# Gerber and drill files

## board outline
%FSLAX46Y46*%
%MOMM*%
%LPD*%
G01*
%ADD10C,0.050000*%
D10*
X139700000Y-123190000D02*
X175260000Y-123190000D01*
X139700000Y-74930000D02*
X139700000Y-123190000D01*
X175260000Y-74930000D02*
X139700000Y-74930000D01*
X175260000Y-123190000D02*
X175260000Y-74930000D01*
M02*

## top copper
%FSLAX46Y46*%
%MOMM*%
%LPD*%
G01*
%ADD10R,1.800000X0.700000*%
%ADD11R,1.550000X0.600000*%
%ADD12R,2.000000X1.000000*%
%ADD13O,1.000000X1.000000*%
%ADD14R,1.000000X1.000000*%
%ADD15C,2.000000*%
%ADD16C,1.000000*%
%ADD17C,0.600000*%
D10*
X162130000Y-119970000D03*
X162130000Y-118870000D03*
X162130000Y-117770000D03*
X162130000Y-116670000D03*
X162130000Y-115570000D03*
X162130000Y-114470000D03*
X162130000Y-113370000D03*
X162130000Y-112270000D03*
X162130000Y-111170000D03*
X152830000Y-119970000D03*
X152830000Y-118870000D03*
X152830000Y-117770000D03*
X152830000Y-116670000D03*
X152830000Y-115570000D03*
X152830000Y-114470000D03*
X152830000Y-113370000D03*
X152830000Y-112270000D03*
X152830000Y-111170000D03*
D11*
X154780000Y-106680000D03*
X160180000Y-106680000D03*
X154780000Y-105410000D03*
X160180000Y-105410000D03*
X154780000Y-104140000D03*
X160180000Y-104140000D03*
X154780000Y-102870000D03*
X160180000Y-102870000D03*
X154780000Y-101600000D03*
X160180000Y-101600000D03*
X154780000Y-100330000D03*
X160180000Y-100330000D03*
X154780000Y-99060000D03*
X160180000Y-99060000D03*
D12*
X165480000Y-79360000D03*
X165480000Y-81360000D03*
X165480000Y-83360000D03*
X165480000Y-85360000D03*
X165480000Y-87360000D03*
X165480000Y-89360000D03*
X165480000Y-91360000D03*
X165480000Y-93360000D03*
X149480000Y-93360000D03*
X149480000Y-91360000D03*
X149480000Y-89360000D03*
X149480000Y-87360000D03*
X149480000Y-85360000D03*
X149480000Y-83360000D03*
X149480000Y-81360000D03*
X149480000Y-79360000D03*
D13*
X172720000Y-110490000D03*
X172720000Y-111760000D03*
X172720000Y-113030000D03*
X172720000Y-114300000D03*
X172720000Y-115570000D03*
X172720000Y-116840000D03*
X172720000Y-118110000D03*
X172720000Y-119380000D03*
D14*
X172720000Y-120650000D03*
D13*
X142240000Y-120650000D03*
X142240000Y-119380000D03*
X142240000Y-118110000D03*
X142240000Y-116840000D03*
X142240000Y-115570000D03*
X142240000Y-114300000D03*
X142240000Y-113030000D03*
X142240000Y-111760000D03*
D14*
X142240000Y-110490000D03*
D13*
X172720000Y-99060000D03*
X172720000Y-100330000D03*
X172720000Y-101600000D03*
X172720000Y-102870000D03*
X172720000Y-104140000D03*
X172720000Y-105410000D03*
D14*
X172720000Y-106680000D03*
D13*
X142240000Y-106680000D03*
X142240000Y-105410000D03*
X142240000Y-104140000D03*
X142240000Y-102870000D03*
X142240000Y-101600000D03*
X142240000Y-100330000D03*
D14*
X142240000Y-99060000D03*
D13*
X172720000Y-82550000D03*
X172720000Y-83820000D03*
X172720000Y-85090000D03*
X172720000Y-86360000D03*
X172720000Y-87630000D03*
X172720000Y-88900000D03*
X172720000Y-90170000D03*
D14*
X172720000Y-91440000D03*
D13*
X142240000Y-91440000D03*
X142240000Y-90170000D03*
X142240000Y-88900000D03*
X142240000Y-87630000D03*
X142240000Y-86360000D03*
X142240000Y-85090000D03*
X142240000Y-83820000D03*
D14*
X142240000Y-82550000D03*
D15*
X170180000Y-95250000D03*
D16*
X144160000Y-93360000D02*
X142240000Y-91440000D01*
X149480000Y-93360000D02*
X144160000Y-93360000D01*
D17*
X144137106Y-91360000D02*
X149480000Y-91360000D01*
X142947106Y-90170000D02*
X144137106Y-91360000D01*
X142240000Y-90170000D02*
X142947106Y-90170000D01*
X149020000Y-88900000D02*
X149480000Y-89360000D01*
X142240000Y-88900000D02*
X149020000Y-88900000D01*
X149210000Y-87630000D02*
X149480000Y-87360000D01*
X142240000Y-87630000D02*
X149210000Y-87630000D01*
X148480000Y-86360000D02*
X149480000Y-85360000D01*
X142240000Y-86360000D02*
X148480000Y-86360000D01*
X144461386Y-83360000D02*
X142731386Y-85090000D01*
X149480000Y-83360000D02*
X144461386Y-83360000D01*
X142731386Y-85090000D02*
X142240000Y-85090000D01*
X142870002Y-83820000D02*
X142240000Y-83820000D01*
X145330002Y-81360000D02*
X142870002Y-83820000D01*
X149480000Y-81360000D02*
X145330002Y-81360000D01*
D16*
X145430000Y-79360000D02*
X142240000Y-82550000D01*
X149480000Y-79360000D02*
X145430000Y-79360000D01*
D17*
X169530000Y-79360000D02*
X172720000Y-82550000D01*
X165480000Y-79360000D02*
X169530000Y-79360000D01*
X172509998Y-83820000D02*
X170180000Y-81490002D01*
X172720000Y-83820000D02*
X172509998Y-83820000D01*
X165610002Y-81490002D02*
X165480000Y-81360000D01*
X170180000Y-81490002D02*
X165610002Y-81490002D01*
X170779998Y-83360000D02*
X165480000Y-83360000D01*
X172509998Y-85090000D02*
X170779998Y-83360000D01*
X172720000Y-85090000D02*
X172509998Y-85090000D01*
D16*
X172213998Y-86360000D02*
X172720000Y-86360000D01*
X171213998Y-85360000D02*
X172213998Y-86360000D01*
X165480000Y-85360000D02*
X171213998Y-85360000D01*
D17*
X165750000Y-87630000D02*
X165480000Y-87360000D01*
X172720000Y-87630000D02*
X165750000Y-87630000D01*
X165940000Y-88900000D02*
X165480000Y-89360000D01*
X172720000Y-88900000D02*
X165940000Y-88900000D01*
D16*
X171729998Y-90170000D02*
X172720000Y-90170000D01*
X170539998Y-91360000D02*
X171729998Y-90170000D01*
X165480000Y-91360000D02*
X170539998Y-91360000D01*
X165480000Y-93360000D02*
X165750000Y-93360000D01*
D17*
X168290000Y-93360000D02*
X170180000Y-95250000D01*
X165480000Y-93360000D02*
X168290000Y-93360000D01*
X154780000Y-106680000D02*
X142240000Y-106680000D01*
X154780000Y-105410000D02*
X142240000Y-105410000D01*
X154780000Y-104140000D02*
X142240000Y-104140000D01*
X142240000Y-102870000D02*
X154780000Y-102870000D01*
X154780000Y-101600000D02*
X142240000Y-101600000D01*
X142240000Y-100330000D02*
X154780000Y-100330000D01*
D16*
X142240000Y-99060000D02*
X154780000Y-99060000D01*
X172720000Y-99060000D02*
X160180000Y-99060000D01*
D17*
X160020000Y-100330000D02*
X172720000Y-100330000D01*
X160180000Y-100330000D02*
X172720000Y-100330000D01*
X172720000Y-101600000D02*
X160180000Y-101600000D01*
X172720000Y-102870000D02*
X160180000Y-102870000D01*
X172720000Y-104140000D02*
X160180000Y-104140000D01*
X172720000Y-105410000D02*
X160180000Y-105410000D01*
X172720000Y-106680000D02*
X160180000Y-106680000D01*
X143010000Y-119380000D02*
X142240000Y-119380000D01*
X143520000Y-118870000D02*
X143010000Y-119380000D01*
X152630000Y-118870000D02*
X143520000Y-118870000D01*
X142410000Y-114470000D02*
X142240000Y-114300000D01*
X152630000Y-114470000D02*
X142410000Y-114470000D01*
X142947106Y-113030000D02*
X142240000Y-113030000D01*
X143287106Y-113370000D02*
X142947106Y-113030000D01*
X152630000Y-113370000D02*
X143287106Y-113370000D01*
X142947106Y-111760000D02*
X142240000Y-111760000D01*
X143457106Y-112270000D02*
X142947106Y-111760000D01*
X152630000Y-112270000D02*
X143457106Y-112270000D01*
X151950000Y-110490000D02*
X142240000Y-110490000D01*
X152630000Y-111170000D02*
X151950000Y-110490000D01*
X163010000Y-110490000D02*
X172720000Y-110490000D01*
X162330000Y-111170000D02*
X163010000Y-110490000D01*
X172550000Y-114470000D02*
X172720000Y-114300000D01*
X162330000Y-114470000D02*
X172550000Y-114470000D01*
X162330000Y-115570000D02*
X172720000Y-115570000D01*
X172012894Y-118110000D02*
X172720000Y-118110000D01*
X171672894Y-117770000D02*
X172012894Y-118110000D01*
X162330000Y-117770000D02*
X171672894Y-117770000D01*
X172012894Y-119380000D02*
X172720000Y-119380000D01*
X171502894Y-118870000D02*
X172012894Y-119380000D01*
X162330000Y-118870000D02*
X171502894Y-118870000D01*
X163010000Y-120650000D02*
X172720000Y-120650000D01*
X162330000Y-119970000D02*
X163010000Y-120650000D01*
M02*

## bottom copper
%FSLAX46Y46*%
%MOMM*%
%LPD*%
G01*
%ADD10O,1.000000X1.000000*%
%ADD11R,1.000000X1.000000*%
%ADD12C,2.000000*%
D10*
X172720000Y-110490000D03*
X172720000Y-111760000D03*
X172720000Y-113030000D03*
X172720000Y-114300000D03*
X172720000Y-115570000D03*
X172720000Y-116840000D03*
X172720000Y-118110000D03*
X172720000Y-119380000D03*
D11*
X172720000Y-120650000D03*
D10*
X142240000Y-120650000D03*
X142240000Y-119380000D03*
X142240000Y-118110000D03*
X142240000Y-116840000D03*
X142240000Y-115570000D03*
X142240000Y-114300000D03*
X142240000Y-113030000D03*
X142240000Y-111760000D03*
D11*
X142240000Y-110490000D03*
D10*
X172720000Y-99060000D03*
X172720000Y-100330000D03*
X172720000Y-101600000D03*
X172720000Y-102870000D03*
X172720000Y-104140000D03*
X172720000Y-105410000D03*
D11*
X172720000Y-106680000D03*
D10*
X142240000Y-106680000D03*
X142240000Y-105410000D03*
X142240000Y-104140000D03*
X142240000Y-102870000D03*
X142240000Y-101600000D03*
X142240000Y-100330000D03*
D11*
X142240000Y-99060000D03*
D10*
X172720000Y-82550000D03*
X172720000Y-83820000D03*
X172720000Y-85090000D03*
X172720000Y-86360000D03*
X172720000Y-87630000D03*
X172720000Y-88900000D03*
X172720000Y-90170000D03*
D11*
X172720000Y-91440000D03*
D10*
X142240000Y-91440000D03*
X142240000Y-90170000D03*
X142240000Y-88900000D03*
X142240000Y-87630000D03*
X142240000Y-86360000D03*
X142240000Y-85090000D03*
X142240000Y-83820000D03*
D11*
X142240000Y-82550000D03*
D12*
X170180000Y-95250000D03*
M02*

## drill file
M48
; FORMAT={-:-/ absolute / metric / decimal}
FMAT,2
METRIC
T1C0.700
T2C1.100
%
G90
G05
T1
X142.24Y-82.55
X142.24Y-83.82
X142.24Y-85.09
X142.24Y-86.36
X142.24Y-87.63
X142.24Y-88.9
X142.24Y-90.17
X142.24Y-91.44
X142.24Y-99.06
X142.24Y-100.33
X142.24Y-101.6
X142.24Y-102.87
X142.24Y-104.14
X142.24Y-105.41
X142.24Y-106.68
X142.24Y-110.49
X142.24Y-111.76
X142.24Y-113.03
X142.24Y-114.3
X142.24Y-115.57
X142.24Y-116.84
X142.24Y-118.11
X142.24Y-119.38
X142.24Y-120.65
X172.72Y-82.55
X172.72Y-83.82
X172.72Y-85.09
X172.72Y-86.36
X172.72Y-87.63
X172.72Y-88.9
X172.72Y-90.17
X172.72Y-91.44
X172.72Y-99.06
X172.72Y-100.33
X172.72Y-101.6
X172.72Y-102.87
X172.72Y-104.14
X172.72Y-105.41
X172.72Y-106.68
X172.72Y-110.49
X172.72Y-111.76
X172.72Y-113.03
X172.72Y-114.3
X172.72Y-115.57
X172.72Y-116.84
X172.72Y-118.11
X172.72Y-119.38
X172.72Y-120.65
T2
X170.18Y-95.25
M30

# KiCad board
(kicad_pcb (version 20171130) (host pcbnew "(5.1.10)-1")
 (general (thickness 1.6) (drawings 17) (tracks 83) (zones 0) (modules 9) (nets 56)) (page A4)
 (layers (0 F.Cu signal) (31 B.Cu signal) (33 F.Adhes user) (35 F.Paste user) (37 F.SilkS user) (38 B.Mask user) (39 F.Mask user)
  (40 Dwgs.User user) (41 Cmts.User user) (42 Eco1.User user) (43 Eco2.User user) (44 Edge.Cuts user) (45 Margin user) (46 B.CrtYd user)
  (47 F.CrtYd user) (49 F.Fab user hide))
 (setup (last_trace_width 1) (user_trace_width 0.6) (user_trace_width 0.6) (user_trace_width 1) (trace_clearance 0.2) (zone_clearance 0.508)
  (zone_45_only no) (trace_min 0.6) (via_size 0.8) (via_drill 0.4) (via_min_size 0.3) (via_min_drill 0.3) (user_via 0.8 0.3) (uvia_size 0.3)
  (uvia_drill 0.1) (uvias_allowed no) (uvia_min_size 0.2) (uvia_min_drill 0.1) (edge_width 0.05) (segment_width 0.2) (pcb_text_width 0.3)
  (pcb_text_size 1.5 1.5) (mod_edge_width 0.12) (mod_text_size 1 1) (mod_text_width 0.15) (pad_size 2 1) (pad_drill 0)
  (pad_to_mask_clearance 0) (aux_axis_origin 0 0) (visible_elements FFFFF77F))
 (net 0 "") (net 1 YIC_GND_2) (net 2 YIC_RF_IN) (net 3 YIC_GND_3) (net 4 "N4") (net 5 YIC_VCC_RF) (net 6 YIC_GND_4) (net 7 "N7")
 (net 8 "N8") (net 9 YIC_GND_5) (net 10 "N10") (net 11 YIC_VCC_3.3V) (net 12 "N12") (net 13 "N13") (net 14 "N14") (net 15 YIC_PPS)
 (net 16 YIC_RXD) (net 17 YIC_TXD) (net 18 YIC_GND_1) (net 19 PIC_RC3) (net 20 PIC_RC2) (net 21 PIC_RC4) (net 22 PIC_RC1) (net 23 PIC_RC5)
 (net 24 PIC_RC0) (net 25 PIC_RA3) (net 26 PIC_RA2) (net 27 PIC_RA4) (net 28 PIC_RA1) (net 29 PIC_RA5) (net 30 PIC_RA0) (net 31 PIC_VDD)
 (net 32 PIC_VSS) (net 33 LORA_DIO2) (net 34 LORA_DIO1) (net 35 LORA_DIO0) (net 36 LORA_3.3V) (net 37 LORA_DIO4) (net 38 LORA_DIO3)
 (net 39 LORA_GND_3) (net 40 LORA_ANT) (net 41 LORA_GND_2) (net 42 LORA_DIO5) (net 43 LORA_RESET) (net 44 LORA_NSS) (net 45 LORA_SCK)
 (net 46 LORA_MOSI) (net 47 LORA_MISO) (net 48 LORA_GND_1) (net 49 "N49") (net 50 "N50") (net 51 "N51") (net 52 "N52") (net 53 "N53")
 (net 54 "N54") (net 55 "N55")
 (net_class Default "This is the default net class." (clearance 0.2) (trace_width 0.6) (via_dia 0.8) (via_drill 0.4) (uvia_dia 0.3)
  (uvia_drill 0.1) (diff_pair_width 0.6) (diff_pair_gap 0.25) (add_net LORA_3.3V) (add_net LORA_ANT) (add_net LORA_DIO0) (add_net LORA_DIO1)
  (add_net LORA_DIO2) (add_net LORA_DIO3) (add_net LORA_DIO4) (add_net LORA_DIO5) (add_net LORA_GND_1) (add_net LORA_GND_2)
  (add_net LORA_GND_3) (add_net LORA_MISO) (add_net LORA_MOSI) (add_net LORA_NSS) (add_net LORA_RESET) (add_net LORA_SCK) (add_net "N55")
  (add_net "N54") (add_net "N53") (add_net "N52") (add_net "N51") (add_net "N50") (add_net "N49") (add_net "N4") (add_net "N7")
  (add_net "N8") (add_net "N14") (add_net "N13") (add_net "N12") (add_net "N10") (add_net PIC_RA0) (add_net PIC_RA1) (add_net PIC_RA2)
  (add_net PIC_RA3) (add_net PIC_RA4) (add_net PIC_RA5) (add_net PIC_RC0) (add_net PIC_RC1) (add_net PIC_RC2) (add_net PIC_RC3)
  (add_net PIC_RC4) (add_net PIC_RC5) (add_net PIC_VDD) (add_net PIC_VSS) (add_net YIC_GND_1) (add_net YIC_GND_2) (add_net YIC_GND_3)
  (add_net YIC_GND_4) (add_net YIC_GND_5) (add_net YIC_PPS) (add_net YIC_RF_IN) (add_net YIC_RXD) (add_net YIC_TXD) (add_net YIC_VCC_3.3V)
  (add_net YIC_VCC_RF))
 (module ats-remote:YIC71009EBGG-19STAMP (layer F.Cu) (at 157.48 115.57 270)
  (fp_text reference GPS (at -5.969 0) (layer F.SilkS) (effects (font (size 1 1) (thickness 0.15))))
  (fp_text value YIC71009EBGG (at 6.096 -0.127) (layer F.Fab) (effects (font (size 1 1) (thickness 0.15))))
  (pad 10 smd rect (at 4.4 -4.85 270) (size 0.7 1.8) (drill (offset 0 0.2)) (layers F.Cu F.Paste F.Mask) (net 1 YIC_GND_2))
  (pad 11 smd rect (at 3.3 -4.85 270) (size 0.7 1.8) (drill (offset 0 0.2)) (layers F.Cu F.Paste F.Mask) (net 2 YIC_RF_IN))
  (pad 12 smd rect (at 2.2 -4.85 270) (size 0.7 1.8) (drill (offset 0 0.2)) (layers F.Cu F.Paste F.Mask) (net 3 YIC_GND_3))
  (pad 13 smd rect (at 1.1 -4.85 270) (size 0.7 1.8) (drill (offset 0 0.2)) (layers F.Cu F.Paste F.Mask) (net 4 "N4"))
  (pad 14 smd rect (at 0 -4.85 270) (size 0.7 1.8) (drill (offset 0 0.2)) (layers F.Cu F.Paste F.Mask) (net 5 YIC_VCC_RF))
  (pad 15 smd rect (at -1.1 -4.85 270) (size 0.7 1.8) (drill (offset 0 0.2)) (layers F.Cu F.Paste F.Mask) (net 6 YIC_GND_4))
  (pad 16 smd rect (at -2.2 -4.85 270) (size 0.7 1.8) (drill (offset 0 0.2)) (layers F.Cu F.Paste F.Mask) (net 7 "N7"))
  (pad 17 smd rect (at -3.3 -4.85 270) (size 0.7 1.8) (drill (offset 0 0.2)) (layers F.Cu F.Paste F.Mask) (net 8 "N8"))
  (pad 18 smd rect (at -4.4 -4.85 270) (size 0.7 1.8) (drill (offset 0 0.2)) (layers F.Cu F.Paste F.Mask) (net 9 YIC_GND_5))
  (pad 9 smd rect (at 4.4 4.85 270) (size 0.7 1.8) (drill (offset 0 -0.2)) (layers F.Cu F.Paste F.Mask) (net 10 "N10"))
  (pad 8 smd rect (at 3.3 4.85 270) (size 0.7 1.8) (drill (offset 0 -0.2)) (layers F.Cu F.Paste F.Mask) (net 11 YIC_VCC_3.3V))
  (pad 7 smd rect (at 2.2 4.85 270) (size 0.7 1.8) (drill (offset 0 -0.2)) (layers F.Cu F.Paste F.Mask) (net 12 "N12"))
  (pad 6 smd rect (at 1.1 4.85 270) (size 0.7 1.8) (drill (offset 0 -0.2)) (layers F.Cu F.Paste F.Mask) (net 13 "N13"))
  (pad 5 smd rect (at 0 4.85 270) (size 0.7 1.8) (drill (offset 0 -0.2)) (layers F.Cu F.Paste F.Mask) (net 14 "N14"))
  (pad 4 smd rect (at -1.1 4.85 270) (size 0.7 1.8) (drill (offset 0 -0.2)) (layers F.Cu F.Paste F.Mask) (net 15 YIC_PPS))
  (pad 3 smd rect (at -2.2 4.85 270) (size 0.7 1.8) (drill (offset 0 -0.2)) (layers F.Cu F.Paste F.Mask) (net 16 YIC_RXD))
  (pad 2 smd rect (at -3.3 4.85 270) (size 0.7 1.8) (drill (offset 0 -0.2)) (layers F.Cu F.Paste F.Mask) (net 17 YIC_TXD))
  (pad 1 smd rect (at -4.4 4.85 270) (size 0.7 1.8) (drill (offset 0 -0.2)) (layers F.Cu F.Paste F.Mask) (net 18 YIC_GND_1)))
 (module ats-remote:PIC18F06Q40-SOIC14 (layer F.Cu) (at 157.48 102.87 270)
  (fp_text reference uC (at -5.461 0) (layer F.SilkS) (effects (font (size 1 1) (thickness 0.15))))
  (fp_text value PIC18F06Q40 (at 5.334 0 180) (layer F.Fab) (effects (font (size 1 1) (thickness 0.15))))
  (pad 7 smd rect (at 3.81 2.7 270) (size 0.6 1.55) (layers F.Cu F.Paste F.Mask) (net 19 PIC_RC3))
  (pad 8 smd rect (at 3.81 -2.7 270) (size 0.6 1.55) (layers F.Cu F.Paste F.Mask) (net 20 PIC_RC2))
  (pad 6 smd rect (at 2.54 2.7 270) (size 0.6 1.55) (layers F.Cu F.Paste F.Mask) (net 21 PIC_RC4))
  (pad 9 smd rect (at 2.54 -2.7 270) (size 0.6 1.55) (layers F.Cu F.Paste F.Mask) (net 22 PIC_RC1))
  (pad 5 smd rect (at 1.27 2.7 270) (size 0.6 1.55) (layers F.Cu F.Paste F.Mask) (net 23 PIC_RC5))
  (pad 10 smd rect (at 1.27 -2.7 270) (size 0.6 1.55) (layers F.Cu F.Paste F.Mask) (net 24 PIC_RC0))
  (pad 4 smd rect (at 0 2.7 270) (size 0.6 1.55) (layers F.Cu F.Paste F.Mask) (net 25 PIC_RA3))
  (pad 11 smd rect (at 0 -2.7 270) (size 0.6 1.55) (layers F.Cu F.Paste F.Mask) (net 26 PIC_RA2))
  (pad 3 smd rect (at -1.27 2.7 270) (size 0.6 1.55) (layers F.Cu F.Paste F.Mask) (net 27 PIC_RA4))
  (pad 12 smd rect (at -1.27 -2.7 270) (size 0.6 1.55) (layers F.Cu F.Paste F.Mask) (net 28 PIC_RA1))
  (pad 2 smd rect (at -2.54 2.7 270) (size 0.6 1.55) (layers F.Cu F.Paste F.Mask) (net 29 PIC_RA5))
  (pad 13 smd rect (at -2.54 -2.7 270) (size 0.6 1.55) (layers F.Cu F.Paste F.Mask) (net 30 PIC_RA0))
  (pad 1 smd rect (at -3.81 2.7 270) (size 0.6 1.55) (layers F.Cu F.Paste F.Mask) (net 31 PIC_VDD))
  (pad 14 smd rect (at -3.81 -2.7 270) (size 0.6 1.55) (layers F.Cu F.Paste F.Mask) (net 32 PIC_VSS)))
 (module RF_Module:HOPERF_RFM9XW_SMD (layer F.Cu) (at 157.48 86.36)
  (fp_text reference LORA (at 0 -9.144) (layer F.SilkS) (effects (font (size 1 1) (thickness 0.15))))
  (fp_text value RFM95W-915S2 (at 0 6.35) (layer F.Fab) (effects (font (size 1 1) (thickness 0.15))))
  (pad 16 smd rect (at 8 -7) (size 2 1) (layers F.Cu F.Paste F.Mask) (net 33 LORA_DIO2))
  (pad 15 smd rect (at 8 -5) (size 2 1) (layers F.Cu F.Paste F.Mask) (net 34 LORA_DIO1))
  (pad 14 smd rect (at 8 -3) (size 2 1) (layers F.Cu F.Paste F.Mask) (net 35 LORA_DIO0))
  (pad 13 smd rect (at 8 -1) (size 2 1) (layers F.Cu F.Paste F.Mask) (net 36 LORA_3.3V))
  (pad 12 smd rect (at 8 1) (size 2 1) (layers F.Cu F.Paste F.Mask) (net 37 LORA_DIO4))
  (pad 11 smd rect (at 8 3) (size 2 1) (layers F.Cu F.Paste F.Mask) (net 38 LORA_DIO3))
  (pad 10 smd rect (at 8 5) (size 2 1) (layers F.Cu F.Paste F.Mask) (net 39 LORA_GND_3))
  (pad 9 smd rect (at 8 7) (size 2 1) (layers F.Cu F.Paste F.Mask) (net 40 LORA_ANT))
  (pad 8 smd rect (at -8 7) (size 2 1) (layers F.Cu F.Paste F.Mask) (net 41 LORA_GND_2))
  (pad 7 smd rect (at -8 5) (size 2 1) (layers F.Cu F.Paste F.Mask) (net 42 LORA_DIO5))
  (pad 6 smd rect (at -8 3) (size 2 1) (layers F.Cu F.Paste F.Mask) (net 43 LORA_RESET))
  (pad 5 smd rect (at -8 1) (size 2 1) (layers F.Cu F.Paste F.Mask) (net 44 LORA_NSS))
  (pad 4 smd rect (at -8 -1) (size 2 1) (layers F.Cu F.Paste F.Mask) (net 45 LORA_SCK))
  (pad 3 smd rect (at -8 -3) (size 2 1) (layers F.Cu F.Paste F.Mask) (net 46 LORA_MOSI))
  (pad 2 smd rect (at -8 -5) (size 2 1) (layers F.Cu F.Paste F.Mask) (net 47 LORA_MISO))
  (pad 1 smd rect (at -8 -7) (size 2 1) (layers F.Cu F.Paste F.Mask) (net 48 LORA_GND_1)))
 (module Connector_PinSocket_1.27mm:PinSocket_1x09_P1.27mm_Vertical (layer F.Cu) (at 172.72 120.65 180)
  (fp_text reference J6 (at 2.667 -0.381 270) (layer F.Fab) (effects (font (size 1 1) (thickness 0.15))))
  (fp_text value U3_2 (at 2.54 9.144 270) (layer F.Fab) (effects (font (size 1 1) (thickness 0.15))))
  (pad 9 thru_hole oval (at 0 10.16 180) (size 1 1) (drill 0.7) (layers *.Cu *.Mask) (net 9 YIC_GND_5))
  (pad 8 thru_hole oval (at 0 8.89 180) (size 1 1) (drill 0.7) (layers *.Cu *.Mask) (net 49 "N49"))
  (pad 7 thru_hole oval (at 0 7.62 180) (size 1 1) (drill 0.7) (layers *.Cu *.Mask) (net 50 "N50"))
  (pad 6 thru_hole oval (at 0 6.35 180) (size 1 1) (drill 0.7) (layers *.Cu *.Mask) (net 6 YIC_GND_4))
  (pad 5 thru_hole oval (at 0 5.08 180) (size 1 1) (drill 0.7) (layers *.Cu *.Mask) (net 5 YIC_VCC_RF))
  (pad 4 thru_hole oval (at 0 3.81 180) (size 1 1) (drill 0.7) (layers *.Cu *.Mask) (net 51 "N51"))
  (pad 3 thru_hole oval (at 0 2.54 180) (size 1 1) (drill 0.7) (layers *.Cu *.Mask) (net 3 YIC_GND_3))
  (pad 2 thru_hole oval (at 0 1.27 180) (size 1 1) (drill 0.7) (layers *.Cu *.Mask) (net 2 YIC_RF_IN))
  (pad 1 thru_hole rect (at 0 0 180) (size 1 1) (drill 0.7) (layers *.Cu *.Mask) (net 1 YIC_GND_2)))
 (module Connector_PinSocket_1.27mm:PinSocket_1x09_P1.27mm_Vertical (layer F.Cu) (at 142.24 110.49)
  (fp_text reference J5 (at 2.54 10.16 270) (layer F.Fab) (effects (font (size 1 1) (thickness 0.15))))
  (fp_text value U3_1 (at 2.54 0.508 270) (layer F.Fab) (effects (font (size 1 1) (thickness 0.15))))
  (pad 9 thru_hole oval (at 0 10.16) (size 1 1) (drill 0.7) (layers *.Cu *.Mask) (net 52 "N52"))
  (pad 8 thru_hole oval (at 0 8.89) (size 1 1) (drill 0.7) (layers *.Cu *.Mask) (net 11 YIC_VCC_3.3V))
  (pad 7 thru_hole oval (at 0 7.62) (size 1 1) (drill 0.7) (layers *.Cu *.Mask) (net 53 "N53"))
  (pad 6 thru_hole oval (at 0 6.35) (size 1 1) (drill 0.7) (layers *.Cu *.Mask) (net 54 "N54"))
  (pad 5 thru_hole oval (at 0 5.08) (size 1 1) (drill 0.7) (layers *.Cu *.Mask) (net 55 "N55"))
  (pad 4 thru_hole oval (at 0 3.81) (size 1 1) (drill 0.7) (layers *.Cu *.Mask) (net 15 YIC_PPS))
  (pad 3 thru_hole oval (at 0 2.54) (size 1 1) (drill 0.7) (layers *.Cu *.Mask) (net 16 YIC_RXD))
  (pad 2 thru_hole oval (at 0 1.27) (size 1 1) (drill 0.7) (layers *.Cu *.Mask) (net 17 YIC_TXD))
  (pad 1 thru_hole rect (at 0 0) (size 1 1) (drill 0.7) (layers *.Cu *.Mask) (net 18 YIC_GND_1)))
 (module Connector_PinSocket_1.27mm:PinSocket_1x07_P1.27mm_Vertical (layer F.Cu) (at 172.72 106.68 180)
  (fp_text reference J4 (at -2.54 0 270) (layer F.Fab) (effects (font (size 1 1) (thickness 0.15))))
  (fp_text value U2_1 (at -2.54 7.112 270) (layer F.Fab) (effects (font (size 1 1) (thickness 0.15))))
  (pad 7 thru_hole oval (at 0 7.62 180) (size 1 1) (drill 0.7) (layers *.Cu *.Mask) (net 32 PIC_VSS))
  (pad 6 thru_hole oval (at 0 6.35 180) (size 1 1) (drill 0.7) (layers *.Cu *.Mask) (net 30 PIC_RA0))
  (pad 5 thru_hole oval (at 0 5.08 180) (size 1 1) (drill 0.7) (layers *.Cu *.Mask) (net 28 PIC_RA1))
  (pad 4 thru_hole oval (at 0 3.81 180) (size 1 1) (drill 0.7) (layers *.Cu *.Mask) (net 26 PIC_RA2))
  (pad 3 thru_hole oval (at 0 2.54 180) (size 1 1) (drill 0.7) (layers *.Cu *.Mask) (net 24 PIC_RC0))
  (pad 2 thru_hole oval (at 0 1.27 180) (size 1 1) (drill 0.7) (layers *.Cu *.Mask) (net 22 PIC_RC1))
  (pad 1 thru_hole rect (at 0 0 180) (size 1 1) (drill 0.7) (layers *.Cu *.Mask) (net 20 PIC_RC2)))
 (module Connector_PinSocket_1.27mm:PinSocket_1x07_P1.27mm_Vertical (layer F.Cu) (at 142.24 99.06)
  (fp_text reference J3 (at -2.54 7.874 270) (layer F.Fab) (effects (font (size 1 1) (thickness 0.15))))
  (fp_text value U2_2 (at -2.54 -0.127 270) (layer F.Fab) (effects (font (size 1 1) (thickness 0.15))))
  (pad 7 thru_hole oval (at 0 7.62) (size 1 1) (drill 0.7) (layers *.Cu *.Mask) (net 19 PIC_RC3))
  (pad 6 thru_hole oval (at 0 6.35) (size 1 1) (drill 0.7) (layers *.Cu *.Mask) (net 21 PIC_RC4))
  (pad 5 thru_hole oval (at 0 5.08) (size 1 1) (drill 0.7) (layers *.Cu *.Mask) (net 23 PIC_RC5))
  (pad 4 thru_hole oval (at 0 3.81) (size 1 1) (drill 0.7) (layers *.Cu *.Mask) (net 25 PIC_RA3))
  (pad 3 thru_hole oval (at 0 2.54) (size 1 1) (drill 0.7) (layers *.Cu *.Mask) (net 27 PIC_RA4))
  (pad 2 thru_hole oval (at 0 1.27) (size 1 1) (drill 0.7) (layers *.Cu *.Mask) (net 29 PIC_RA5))
  (pad 1 thru_hole rect (at 0 0) (size 1 1) (drill 0.7) (layers *.Cu *.Mask) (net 31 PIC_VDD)))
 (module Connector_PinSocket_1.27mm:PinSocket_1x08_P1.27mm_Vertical (layer F.Cu) (at 172.72 91.44 180)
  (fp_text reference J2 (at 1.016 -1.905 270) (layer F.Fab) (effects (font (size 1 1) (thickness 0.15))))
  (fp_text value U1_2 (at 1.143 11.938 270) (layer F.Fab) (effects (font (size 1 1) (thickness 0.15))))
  (pad 8 thru_hole oval (at 0 8.89 180) (size 1 1) (drill 0.7) (layers *.Cu *.Mask) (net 33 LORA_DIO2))
  (pad 7 thru_hole oval (at 0 7.62 180) (size 1 1) (drill 0.7) (layers *.Cu *.Mask) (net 34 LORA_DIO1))
  (pad 6 thru_hole oval (at 0 6.35 180) (size 1 1) (drill 0.7) (layers *.Cu *.Mask) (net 35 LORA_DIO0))
  (pad 5 thru_hole oval (at 0 5.08 180) (size 1 1) (drill 0.7) (layers *.Cu *.Mask) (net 36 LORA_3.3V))
  (pad 4 thru_hole oval (at 0 3.81 180) (size 1 1) (drill 0.7) (layers *.Cu *.Mask) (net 37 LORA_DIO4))
  (pad 3 thru_hole oval (at 0 2.54 180) (size 1 1) (drill 0.7) (layers *.Cu *.Mask) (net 38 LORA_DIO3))
  (pad 2 thru_hole oval (at 0 1.27 180) (size 1 1) (drill 0.7) (layers *.Cu *.Mask) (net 39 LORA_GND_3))
  (pad 1 thru_hole rect (at 0 0 180) (size 1 1) (drill 0.7) (layers *.Cu *.Mask) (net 40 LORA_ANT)))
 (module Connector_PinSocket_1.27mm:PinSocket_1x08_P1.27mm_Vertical (layer F.Cu) (at 142.24 82.55)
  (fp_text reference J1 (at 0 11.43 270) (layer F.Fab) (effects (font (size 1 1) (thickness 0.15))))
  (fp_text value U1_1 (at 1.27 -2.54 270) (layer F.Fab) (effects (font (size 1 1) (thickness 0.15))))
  (pad 8 thru_hole oval (at 0 8.89) (size 1 1) (drill 0.7) (layers *.Cu *.Mask) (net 41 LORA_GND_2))
  (pad 7 thru_hole oval (at 0 7.62) (size 1 1) (drill 0.7) (layers *.Cu *.Mask) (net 42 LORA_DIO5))
  (pad 6 thru_hole oval (at 0 6.35) (size 1 1) (drill 0.7) (layers *.Cu *.Mask) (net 43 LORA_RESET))
  (pad 5 thru_hole oval (at 0 5.08) (size 1 1) (drill 0.7) (layers *.Cu *.Mask) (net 44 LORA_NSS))
  (pad 4 thru_hole oval (at 0 3.81) (size 1 1) (drill 0.7) (layers *.Cu *.Mask) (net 45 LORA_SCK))
  (pad 3 thru_hole oval (at 0 2.54) (size 1 1) (drill 0.7) (layers *.Cu *.Mask) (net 46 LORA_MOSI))
  (pad 2 thru_hole oval (at 0 1.27) (size 1 1) (drill 0.7) (layers *.Cu *.Mask) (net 47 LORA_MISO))
  (pad 1 thru_hole rect (at 0 0) (size 1 1) (drill 0.7) (layers *.Cu *.Mask) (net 48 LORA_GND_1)))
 (gr_line (start 139.7 123.19) (end 175.26 123.19) (layer Edge.Cuts) (width 0.05))
 (gr_line (start 139.7 74.93) (end 139.7 123.19) (layer Edge.Cuts) (width 0.05))
 (gr_line (start 175.26 74.93) (end 139.7 74.93) (layer Edge.Cuts) (width 0.05))
 (gr_line (start 175.26 123.19) (end 175.26 74.93) (layer Edge.Cuts) (width 0.05))
 (segment (start 144.16 93.36) (end 142.24 91.44) (width 1) (layer F.Cu) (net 41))
 (segment (start 149.48 93.36) (end 144.16 93.36) (width 1) (layer F.Cu) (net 41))
 (segment (start 144.137106 91.36) (end 149.48 91.36) (width 0.6) (layer F.Cu) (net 42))
 (segment (start 142.947106 90.17) (end 144.137106 91.36) (width 0.6) (layer F.Cu) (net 42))
 (segment (start 142.24 90.17) (end 142.947106 90.17) (width 0.6) (layer F.Cu) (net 42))
 (segment (start 149.02 88.9) (end 149.48 89.36) (width 0.6) (layer F.Cu) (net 43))
 (segment (start 142.24 88.9) (end 149.02 88.9) (width 0.6) (layer F.Cu) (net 43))
 (via (at 170.18 95.25) (size 2) (drill 1.1) (layers F.Cu B.Cu) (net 40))
 (segment (start 149.21 87.63) (end 149.48 87.36) (width 0.6) (layer F.Cu) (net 44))
 (segment (start 142.24 87.63) (end 149.21 87.63) (width 0.6) (layer F.Cu) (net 44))
 (segment (start 148.48 86.36) (end 149.48 85.36) (width 0.6) (layer F.Cu) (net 45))
 (segment (start 142.24 86.36) (end 148.48 86.36) (width 0.6) (layer F.Cu) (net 45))
 (segment (start 144.461386 83.36) (end 142.731386 85.09) (width 0.6) (layer F.Cu) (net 46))
 (segment (start 149.48 83.36) (end 144.461386 83.36) (width 0.6) (layer F.Cu) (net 46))
 (segment (start 142.731386 85.09) (end 142.24 85.09) (width 0.6) (layer F.Cu) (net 46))
 (segment (start 142.870002 83.82) (end 142.24 83.82) (width 0.6) (layer F.Cu) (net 47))
 (segment (start 145.330002 81.36) (end 142.870002 83.82) (width 0.6) (layer F.Cu) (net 47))
 (segment (start 149.48 81.36) (end 145.330002 81.36) (width 0.6) (layer F.Cu) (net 47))
 (segment (start 145.43 79.36) (end 142.24 82.55) (width 1) (layer F.Cu) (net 48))
 (segment (start 149.48 79.36) (end 145.43 79.36) (width 1) (layer F.Cu) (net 48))
 (segment (start 169.53 79.36) (end 172.72 82.55) (width 0.6) (layer F.Cu) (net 33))
 (segment (start 165.48 79.36) (end 169.53 79.36) (width 0.6) (layer F.Cu) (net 33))
 (segment (start 172.509998 83.82) (end 170.18 81.490002) (width 0.6) (layer F.Cu) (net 34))
 (segment (start 172.72 83.82) (end 172.509998 83.82) (width 0.6) (layer F.Cu) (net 34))
 (segment (start 165.610002 81.490002) (end 165.48 81.36) (width 0.6) (layer F.Cu) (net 34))
 (segment (start 170.18 81.490002) (end 165.610002 81.490002) (width 0.6) (layer F.Cu) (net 34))
 (segment (start 170.779998 83.36) (end 165.48 83.36) (width 0.6) (layer F.Cu) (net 35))
 (segment (start 172.509998 85.09) (end 170.779998 83.36) (width 0.6) (layer F.Cu) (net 35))
 (segment (start 172.72 85.09) (end 172.509998 85.09) (width 0.6) (layer F.Cu) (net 35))
 (segment (start 172.213998 86.36) (end 172.72 86.36) (width 1) (layer F.Cu) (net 36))
 (segment (start 171.213998 85.36) (end 172.213998 86.36) (width 1) (layer F.Cu) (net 36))
 (segment (start 165.48 85.36) (end 171.213998 85.36) (width 1) (layer F.Cu) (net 36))
 (segment (start 165.75 87.63) (end 165.48 87.36) (width 0.6) (layer F.Cu) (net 37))
 (segment (start 172.72 87.63) (end 165.75 87.63) (width 0.6) (layer F.Cu) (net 37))
 (segment (start 165.94 88.9) (end 165.48 89.36) (width 0.6) (layer F.Cu) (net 38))
 (segment (start 172.72 88.9) (end 165.94 88.9) (width 0.6) (layer F.Cu) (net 38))
 (segment (start 171.729998 90.17) (end 172.72 90.17) (width 1) (layer F.Cu) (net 39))
 (segment (start 170.539998 91.36) (end 171.729998 90.17) (width 1) (layer F.Cu) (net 39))
 (segment (start 165.48 91.36) (end 170.539998 91.36) (width 1) (layer F.Cu) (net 39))
 (segment (start 165.48 93.36) (end 165.75 93.36) (width 1) (layer F.Cu) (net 40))
 (segment (start 168.29 93.36) (end 170.18 95.25) (width 0.6) (layer F.Cu) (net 40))
 (segment (start 165.48 93.36) (end 168.29 93.36) (width 0.6) (layer F.Cu) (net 40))
 (segment (start 154.78 106.68) (end 142.24 106.68) (width 0.6) (layer F.Cu) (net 19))
 (segment (start 154.78 105.41) (end 142.24 105.41) (width 0.6) (layer F.Cu) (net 21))
 (segment (start 154.78 104.14) (end 142.24 104.14) (width 0.6) (layer F.Cu) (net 23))
 (segment (start 142.24 102.87) (end 154.78 102.87) (width 0.6) (layer F.Cu) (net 25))
 (segment (start 154.78 101.6) (end 142.24 101.6) (width 0.6) (layer F.Cu) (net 27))
 (segment (start 142.24 100.33) (end 154.78 100.33) (width 0.6) (layer F.Cu) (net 29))
 (segment (start 142.24 99.06) (end 154.78 99.06) (width 1) (layer F.Cu) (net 31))
 (segment (start 172.72 99.06) (end 160.18 99.06) (width 1) (layer F.Cu) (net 32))
 (segment (start 160.02 100.33) (end 172.72 100.33) (width 0.6) (layer F.Cu) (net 30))
 (segment (start 160.18 100.33) (end 172.72 100.33) (width 0.6) (layer F.Cu) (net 30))
 (segment (start 172.72 101.6) (end 160.18 101.6) (width 0.6) (layer F.Cu) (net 28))
 (segment (start 172.72 102.87) (end 160.18 102.87) (width 0.6) (layer F.Cu) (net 26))
 (segment (start 172.72 104.14) (end 160.18 104.14) (width 0.6) (layer F.Cu) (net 24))
 (segment (start 172.72 105.41) (end 160.18 105.41) (width 0.6) (layer F.Cu) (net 22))
 (segment (start 172.72 106.68) (end 160.18 106.68) (width 0.6) (layer F.Cu) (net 20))
 (segment (start 143.01 119.38) (end 142.24 119.38) (width 0.6) (layer F.Cu) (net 11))
 (segment (start 143.52 118.87) (end 143.01 119.38) (width 0.6) (layer F.Cu) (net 11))
 (segment (start 152.63 118.87) (end 143.52 118.87) (width 0.6) (layer F.Cu) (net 11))
 (segment (start 142.41 114.47) (end 142.24 114.3) (width 0.6) (layer F.Cu) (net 15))
 (segment (start 152.63 114.47) (end 142.41 114.47) (width 0.6) (layer F.Cu) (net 15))
 (segment (start 142.947106 113.03) (end 142.24 113.03) (width 0.6) (layer F.Cu) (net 16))
 (segment (start 143.287106 113.37) (end 142.947106 113.03) (width 0.6) (layer F.Cu) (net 16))
 (segment (start 152.63 113.37) (end 143.287106 113.37) (width 0.6) (layer F.Cu) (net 16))
 (segment (start 142.947106 111.76) (end 142.24 111.76) (width 0.6) (layer F.Cu) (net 17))
 (segment (start 143.457106 112.27) (end 142.947106 111.76) (width 0.6) (layer F.Cu) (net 17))
 (segment (start 152.63 112.27) (end 143.457106 112.27) (width 0.6) (layer F.Cu) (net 17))
 (segment (start 151.95 110.49) (end 142.24 110.49) (width 0.6) (layer F.Cu) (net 18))
 (segment (start 152.63 111.17) (end 151.95 110.49) (width 0.6) (layer F.Cu) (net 18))
 (segment (start 163.01 110.49) (end 172.72 110.49) (width 0.6) (layer F.Cu) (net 9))
 (segment (start 162.33 111.17) (end 163.01 110.49) (width 0.6) (layer F.Cu) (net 9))
 (segment (start 172.55 114.47) (end 172.72 114.3) (width 0.6) (layer F.Cu) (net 6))
 (segment (start 162.33 114.47) (end 172.55 114.47) (width 0.6) (layer F.Cu) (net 6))
 (segment (start 162.33 115.57) (end 172.72 115.57) (width 0.6) (layer F.Cu) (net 5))
 (segment (start 172.012894 118.11) (end 172.72 118.11) (width 0.6) (layer F.Cu) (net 3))
 (segment (start 171.672894 117.77) (end 172.012894 118.11) (width 0.6) (layer F.Cu) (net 3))
 (segment (start 162.33 117.77) (end 171.672894 117.77) (width 0.6) (layer F.Cu) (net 3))
 (segment (start 172.012894 119.38) (end 172.72 119.38) (width 0.6) (layer F.Cu) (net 2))
 (segment (start 171.502894 118.87) (end 172.012894 119.38) (width 0.6) (layer F.Cu) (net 2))
 (segment (start 162.33 118.87) (end 171.502894 118.87) (width 0.6) (layer F.Cu) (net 2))
 (segment (start 163.01 120.65) (end 172.72 120.65) (width 0.6) (layer F.Cu) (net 1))
 (segment (start 162.33 119.97) (end 163.01 120.65) (width 0.6) (layer F.Cu) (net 1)))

